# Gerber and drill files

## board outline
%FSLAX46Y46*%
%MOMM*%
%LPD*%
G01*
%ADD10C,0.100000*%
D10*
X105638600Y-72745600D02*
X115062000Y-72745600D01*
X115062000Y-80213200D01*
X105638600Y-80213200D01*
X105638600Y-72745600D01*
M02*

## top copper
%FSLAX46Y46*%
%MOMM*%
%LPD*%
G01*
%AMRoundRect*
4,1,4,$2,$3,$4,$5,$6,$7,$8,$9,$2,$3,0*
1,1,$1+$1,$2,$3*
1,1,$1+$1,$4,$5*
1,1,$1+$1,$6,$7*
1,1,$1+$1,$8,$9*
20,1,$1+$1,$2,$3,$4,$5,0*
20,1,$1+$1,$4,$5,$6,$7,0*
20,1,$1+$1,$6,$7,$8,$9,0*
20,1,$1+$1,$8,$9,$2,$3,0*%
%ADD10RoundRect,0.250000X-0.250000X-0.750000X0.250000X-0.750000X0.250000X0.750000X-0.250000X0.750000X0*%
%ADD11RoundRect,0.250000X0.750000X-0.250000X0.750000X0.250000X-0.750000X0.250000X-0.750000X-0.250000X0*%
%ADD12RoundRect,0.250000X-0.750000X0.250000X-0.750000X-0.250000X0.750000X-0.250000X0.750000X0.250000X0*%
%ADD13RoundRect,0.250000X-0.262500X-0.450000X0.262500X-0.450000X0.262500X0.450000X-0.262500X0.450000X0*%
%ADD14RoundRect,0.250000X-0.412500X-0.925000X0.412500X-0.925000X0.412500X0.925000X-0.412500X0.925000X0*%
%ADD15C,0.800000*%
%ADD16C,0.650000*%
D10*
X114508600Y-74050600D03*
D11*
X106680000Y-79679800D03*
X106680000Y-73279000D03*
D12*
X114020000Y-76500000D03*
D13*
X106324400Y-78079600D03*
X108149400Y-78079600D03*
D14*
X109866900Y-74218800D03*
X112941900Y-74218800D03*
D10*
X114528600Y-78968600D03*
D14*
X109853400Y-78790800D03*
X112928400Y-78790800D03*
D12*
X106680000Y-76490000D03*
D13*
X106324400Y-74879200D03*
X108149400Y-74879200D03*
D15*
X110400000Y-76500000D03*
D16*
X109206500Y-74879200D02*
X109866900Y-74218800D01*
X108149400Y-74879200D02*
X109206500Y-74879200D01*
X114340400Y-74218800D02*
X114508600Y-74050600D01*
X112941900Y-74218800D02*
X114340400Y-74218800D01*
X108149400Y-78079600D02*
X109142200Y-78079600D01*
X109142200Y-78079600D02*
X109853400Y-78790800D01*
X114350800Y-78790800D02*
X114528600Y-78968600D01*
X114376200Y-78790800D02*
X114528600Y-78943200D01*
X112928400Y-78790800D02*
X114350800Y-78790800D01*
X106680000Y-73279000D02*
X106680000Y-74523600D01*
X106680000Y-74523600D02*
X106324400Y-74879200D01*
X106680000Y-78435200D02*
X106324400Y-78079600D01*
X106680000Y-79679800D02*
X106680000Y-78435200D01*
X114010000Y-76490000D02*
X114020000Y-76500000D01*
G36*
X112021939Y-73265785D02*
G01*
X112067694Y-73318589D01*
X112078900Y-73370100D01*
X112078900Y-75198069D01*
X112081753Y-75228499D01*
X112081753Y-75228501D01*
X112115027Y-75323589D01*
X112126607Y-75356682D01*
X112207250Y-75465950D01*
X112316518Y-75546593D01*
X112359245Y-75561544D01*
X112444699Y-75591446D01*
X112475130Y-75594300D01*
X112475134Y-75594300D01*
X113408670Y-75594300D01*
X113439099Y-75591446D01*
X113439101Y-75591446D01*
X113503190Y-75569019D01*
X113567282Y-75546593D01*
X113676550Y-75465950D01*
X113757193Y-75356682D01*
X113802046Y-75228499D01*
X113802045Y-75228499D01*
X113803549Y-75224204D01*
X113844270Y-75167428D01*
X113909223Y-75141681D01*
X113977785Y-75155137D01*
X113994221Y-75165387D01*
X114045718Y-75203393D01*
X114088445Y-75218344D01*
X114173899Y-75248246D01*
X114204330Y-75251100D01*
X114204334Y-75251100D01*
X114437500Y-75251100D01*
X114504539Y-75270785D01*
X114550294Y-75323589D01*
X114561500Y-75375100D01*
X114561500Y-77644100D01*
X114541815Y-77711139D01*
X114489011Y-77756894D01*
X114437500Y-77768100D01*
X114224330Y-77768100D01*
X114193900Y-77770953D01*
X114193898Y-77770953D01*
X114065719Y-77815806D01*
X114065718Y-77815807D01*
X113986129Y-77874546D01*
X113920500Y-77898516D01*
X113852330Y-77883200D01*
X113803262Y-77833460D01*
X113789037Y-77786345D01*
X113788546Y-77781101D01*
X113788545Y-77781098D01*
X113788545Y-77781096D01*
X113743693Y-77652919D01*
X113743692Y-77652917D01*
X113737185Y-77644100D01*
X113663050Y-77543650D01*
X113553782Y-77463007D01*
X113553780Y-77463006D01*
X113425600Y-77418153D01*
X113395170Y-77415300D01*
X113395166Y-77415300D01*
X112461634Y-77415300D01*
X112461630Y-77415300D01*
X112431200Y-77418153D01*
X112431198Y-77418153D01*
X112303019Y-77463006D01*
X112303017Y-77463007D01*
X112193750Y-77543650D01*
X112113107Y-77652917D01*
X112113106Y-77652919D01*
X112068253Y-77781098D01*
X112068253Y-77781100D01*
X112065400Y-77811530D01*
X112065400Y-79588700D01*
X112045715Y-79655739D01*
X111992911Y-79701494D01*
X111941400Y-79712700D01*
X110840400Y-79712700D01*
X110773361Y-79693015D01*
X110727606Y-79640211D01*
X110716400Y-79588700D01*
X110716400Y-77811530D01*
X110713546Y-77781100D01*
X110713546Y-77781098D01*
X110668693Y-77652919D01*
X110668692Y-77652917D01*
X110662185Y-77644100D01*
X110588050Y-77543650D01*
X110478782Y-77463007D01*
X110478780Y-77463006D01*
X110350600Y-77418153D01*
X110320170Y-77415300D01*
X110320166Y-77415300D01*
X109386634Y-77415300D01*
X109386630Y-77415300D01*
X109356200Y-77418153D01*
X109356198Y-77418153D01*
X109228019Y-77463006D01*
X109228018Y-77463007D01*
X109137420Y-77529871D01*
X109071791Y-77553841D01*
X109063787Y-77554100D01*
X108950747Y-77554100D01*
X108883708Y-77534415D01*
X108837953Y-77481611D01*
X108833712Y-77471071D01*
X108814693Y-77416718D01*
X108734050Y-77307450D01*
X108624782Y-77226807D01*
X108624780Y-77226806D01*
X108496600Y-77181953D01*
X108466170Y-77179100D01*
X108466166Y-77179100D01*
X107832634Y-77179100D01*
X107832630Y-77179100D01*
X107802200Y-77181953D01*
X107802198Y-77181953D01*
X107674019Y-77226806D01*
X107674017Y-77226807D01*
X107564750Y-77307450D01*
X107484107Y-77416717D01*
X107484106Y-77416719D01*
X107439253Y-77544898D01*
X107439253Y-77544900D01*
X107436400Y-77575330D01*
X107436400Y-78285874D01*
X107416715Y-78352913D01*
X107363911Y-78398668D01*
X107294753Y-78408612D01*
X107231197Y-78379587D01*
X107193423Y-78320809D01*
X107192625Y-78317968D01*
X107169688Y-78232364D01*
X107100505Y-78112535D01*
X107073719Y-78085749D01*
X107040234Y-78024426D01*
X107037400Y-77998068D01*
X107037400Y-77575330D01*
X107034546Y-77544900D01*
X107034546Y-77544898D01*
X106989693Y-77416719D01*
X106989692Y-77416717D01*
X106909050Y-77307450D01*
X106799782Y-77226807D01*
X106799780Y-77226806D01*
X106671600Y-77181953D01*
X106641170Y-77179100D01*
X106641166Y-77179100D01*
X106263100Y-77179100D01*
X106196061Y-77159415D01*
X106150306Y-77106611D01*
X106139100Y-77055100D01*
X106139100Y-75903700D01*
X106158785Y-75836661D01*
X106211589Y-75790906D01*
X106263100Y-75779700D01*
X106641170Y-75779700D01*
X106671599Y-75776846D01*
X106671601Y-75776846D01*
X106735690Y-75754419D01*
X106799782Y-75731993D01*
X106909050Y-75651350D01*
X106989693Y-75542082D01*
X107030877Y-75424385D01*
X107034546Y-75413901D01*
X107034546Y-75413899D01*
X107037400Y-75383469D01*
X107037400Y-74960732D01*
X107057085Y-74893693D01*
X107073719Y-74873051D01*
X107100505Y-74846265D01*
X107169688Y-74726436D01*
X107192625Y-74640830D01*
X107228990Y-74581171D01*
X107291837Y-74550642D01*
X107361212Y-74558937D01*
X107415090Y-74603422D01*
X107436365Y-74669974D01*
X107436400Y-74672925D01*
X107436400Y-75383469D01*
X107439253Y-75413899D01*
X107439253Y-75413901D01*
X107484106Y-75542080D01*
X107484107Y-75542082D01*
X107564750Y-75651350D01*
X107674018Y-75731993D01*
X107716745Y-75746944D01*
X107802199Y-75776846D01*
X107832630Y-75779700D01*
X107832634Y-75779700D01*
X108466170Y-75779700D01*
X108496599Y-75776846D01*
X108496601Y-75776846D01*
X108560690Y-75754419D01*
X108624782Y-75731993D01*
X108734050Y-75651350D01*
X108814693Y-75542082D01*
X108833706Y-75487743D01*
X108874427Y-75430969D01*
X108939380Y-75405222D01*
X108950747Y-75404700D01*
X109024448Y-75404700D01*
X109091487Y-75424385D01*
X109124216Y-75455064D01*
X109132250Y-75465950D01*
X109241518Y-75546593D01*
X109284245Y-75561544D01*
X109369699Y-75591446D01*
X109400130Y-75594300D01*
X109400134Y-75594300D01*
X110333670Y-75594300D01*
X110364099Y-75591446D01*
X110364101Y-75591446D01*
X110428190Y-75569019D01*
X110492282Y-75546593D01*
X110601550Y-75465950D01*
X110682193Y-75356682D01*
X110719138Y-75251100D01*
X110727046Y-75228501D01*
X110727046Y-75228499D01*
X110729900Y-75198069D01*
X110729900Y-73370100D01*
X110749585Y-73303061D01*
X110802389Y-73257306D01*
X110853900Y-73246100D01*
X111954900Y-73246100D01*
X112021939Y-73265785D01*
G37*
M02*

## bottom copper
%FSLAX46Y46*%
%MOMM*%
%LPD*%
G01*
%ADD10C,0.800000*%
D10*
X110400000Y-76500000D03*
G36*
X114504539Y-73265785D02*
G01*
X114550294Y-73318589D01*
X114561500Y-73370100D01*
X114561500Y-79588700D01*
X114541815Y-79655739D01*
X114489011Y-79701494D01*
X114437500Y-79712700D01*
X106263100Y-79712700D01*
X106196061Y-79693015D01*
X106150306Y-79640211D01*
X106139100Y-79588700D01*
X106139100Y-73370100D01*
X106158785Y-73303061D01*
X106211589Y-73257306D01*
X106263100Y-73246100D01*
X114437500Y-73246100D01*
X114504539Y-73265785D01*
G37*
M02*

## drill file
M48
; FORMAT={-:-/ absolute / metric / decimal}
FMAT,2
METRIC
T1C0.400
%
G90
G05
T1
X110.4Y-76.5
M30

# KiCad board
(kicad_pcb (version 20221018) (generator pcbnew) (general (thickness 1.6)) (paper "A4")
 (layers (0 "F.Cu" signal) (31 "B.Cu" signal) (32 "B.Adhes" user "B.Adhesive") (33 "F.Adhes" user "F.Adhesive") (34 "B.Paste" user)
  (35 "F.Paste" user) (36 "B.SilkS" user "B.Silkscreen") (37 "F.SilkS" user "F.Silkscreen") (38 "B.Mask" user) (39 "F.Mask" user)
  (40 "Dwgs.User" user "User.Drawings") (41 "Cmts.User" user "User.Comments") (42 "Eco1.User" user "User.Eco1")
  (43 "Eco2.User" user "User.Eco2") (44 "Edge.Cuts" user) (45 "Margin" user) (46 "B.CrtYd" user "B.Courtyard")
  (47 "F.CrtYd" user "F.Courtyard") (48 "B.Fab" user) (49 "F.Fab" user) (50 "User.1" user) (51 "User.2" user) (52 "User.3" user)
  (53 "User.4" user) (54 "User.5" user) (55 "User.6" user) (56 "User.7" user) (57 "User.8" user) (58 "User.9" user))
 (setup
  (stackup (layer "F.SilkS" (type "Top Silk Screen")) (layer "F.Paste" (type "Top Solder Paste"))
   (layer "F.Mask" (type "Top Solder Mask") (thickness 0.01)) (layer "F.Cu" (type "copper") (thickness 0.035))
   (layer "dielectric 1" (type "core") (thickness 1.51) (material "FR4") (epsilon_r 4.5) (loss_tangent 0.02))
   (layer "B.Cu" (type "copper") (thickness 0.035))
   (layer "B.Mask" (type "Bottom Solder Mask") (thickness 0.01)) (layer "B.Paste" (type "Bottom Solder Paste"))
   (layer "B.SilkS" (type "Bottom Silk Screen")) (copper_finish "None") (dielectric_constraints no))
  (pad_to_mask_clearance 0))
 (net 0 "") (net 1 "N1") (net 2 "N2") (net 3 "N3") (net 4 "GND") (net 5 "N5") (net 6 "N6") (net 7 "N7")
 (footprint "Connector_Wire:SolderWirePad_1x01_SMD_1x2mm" (layer "F.Cu") (at 114.5086 74.0506)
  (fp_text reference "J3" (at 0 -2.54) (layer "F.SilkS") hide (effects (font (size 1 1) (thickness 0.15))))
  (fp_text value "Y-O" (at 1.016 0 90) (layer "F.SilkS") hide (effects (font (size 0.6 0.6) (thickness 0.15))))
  (pad "1" smd roundrect (at 0 0) (size 1 2) (layers "F.Cu" "F.Paste" "F.Mask") (roundrect_rratio 0.25) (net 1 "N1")))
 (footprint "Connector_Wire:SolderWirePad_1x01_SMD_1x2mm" (layer "F.Cu") (at 106.68 79.6798 90)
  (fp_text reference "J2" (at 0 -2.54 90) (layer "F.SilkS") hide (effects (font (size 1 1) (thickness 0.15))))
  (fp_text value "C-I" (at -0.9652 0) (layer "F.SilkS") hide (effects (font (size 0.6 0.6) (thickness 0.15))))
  (pad "1" smd roundrect (at 0 0 90) (size 1 2) (layers "F.Cu" "F.Paste" "F.Mask") (roundrect_rratio 0.25) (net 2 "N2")))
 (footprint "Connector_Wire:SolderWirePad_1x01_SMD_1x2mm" (layer "F.Cu") (at 106.68 73.279 90)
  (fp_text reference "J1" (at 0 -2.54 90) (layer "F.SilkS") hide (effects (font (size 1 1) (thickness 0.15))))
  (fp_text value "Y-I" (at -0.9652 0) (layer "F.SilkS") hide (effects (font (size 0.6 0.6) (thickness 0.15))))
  (pad "1" smd roundrect (at 0 0 90) (size 1 2) (layers "F.Cu" "F.Paste" "F.Mask") (roundrect_rratio 0.25) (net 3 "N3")))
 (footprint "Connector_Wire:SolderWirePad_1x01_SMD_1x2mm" (layer "F.Cu") (at 114.02 76.5 -90)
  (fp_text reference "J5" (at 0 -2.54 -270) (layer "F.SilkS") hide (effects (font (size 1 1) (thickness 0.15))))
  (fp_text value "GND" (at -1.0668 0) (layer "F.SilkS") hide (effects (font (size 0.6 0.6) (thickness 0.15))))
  (pad "1" smd roundrect (at 0 0 270) (size 1 2) (layers "F.Cu" "F.Paste" "F.Mask") (roundrect_rratio 0.25) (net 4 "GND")))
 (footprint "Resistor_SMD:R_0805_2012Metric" (layer "F.Cu") (at 107.2369 78.0796)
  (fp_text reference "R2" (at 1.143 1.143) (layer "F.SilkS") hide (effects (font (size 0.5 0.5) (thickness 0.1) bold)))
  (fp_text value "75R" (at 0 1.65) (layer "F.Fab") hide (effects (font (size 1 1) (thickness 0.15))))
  (pad "1" smd roundrect (at -0.9125 0) (size 1.025 1.4) (layers "F.Cu" "F.Paste" "F.Mask") (roundrect_rratio 0.243902439) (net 2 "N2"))
  (pad "2" smd roundrect (at 0.9125 0) (size 1.025 1.4) (layers "F.Cu" "F.Paste" "F.Mask") (roundrect_rratio 0.243902439) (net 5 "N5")))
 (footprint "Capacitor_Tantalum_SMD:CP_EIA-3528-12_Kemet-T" (layer "F.Cu") (at 111.4044 74.2188)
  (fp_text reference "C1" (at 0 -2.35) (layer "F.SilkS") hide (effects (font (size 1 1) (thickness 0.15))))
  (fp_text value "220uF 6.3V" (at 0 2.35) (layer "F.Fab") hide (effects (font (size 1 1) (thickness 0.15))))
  (pad "1" smd roundrect (at -1.5375 0) (size 1.325 2.35) (layers "F.Cu" "F.Paste" "F.Mask") (roundrect_rratio 0.1886792453) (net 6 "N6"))
  (pad "2" smd roundrect (at 1.5375 0) (size 1.325 2.35) (layers "F.Cu" "F.Paste" "F.Mask") (roundrect_rratio 0.1886792453) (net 1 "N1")))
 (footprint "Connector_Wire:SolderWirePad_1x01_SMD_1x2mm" (layer "F.Cu") (at 114.5286 78.9686)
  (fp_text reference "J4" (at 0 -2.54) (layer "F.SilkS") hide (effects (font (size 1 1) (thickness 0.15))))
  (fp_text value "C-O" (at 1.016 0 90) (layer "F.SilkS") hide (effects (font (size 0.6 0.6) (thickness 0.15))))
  (pad "1" smd roundrect (at 0 0) (size 1 2) (layers "F.Cu" "F.Paste" "F.Mask") (roundrect_rratio 0.25) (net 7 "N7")))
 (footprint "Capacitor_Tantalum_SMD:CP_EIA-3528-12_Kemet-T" (layer "F.Cu") (at 111.3909 78.7908)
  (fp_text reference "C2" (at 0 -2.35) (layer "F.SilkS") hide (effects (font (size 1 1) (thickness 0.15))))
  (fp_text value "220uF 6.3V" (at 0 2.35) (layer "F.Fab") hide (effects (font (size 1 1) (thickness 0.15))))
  (pad "1" smd roundrect (at -1.5375 0) (size 1.325 2.35) (layers "F.Cu" "F.Paste" "F.Mask") (roundrect_rratio 0.1886792453) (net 5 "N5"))
  (pad "2" smd roundrect (at 1.5375 0) (size 1.325 2.35) (layers "F.Cu" "F.Paste" "F.Mask") (roundrect_rratio 0.1886792453) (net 7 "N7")))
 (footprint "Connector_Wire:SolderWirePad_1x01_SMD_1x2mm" (layer "F.Cu") (at 106.68 76.49 -90)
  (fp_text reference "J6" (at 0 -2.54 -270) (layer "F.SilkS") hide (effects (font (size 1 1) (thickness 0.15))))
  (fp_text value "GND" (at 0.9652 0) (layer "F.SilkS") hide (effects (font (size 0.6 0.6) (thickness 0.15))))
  (pad "1" smd roundrect (at 0 0 270) (size 1 2) (layers "F.Cu" "F.Paste" "F.Mask") (roundrect_rratio 0.25) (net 4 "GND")))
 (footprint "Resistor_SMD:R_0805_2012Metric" (layer "F.Cu") (at 107.2369 74.8792)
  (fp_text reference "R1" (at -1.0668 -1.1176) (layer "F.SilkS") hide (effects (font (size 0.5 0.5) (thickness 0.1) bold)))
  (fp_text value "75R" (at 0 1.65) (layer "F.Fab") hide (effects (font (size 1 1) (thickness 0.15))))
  (pad "1" smd roundrect (at -0.9125 0) (size 1.025 1.4) (layers "F.Cu" "F.Paste" "F.Mask") (roundrect_rratio 0.243902439) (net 3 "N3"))
  (pad "2" smd roundrect (at 0.9125 0) (size 1.025 1.4) (layers "F.Cu" "F.Paste" "F.Mask") (roundrect_rratio 0.243902439) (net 6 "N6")))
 (gr_rect (start 105.6386 72.7456) (end 115.062 80.2132) (stroke (width 0.1) (type default)) (fill none) (layer "Edge.Cuts"))
 (segment (start 109.2065 74.8792) (end 109.8669 74.2188) (width 0.65) (layer "F.Cu") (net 6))
 (segment (start 108.1494 74.8792) (end 109.2065 74.8792) (width 0.65) (layer "F.Cu") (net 6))
 (segment (start 114.3404 74.2188) (end 114.5086 74.0506) (width 0.65) (layer "F.Cu") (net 1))
 (segment (start 112.9419 74.2188) (end 114.3404 74.2188) (width 0.65) (layer "F.Cu") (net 1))
 (segment (start 108.1494 78.0796) (end 109.1422 78.0796) (width 0.65) (layer "F.Cu") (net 5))
 (segment (start 109.1422 78.0796) (end 109.8534 78.7908) (width 0.65) (layer "F.Cu") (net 5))
 (segment (start 114.3508 78.7908) (end 114.5286 78.9686) (width 0.65) (layer "F.Cu") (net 7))
 (segment (start 114.3762 78.7908) (end 114.5286 78.9432) (width 0.65) (layer "F.Cu") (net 7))
 (segment (start 112.9284 78.7908) (end 114.3508 78.7908) (width 0.65) (layer "F.Cu") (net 7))
 (segment (start 106.68 73.279) (end 106.68 74.5236) (width 0.65) (layer "F.Cu") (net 3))
 (segment (start 106.68 74.5236) (end 106.3244 74.8792) (width 0.65) (layer "F.Cu") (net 3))
 (segment (start 106.68 78.4352) (end 106.3244 78.0796) (width 0.65) (layer "F.Cu") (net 2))
 (segment (start 106.68 79.6798) (end 106.68 78.4352) (width 0.65) (layer "F.Cu") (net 2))
 (segment (start 114.01 76.49) (end 114.02 76.5) (width 0.65) (layer "F.Cu") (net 4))
 (via (at 110.4 76.5) (size 0.8) (drill 0.4) (layers "F.Cu" "B.Cu") (free) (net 4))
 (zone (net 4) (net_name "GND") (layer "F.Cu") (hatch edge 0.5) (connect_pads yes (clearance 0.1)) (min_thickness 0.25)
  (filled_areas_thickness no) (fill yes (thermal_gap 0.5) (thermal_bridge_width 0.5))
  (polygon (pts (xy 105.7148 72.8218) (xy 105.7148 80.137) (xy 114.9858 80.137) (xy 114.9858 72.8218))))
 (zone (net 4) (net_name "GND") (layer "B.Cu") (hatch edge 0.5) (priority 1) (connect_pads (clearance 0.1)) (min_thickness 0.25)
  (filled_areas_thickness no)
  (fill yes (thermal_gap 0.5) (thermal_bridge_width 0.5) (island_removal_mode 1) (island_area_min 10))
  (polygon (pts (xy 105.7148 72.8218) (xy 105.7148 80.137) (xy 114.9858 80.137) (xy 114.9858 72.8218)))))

